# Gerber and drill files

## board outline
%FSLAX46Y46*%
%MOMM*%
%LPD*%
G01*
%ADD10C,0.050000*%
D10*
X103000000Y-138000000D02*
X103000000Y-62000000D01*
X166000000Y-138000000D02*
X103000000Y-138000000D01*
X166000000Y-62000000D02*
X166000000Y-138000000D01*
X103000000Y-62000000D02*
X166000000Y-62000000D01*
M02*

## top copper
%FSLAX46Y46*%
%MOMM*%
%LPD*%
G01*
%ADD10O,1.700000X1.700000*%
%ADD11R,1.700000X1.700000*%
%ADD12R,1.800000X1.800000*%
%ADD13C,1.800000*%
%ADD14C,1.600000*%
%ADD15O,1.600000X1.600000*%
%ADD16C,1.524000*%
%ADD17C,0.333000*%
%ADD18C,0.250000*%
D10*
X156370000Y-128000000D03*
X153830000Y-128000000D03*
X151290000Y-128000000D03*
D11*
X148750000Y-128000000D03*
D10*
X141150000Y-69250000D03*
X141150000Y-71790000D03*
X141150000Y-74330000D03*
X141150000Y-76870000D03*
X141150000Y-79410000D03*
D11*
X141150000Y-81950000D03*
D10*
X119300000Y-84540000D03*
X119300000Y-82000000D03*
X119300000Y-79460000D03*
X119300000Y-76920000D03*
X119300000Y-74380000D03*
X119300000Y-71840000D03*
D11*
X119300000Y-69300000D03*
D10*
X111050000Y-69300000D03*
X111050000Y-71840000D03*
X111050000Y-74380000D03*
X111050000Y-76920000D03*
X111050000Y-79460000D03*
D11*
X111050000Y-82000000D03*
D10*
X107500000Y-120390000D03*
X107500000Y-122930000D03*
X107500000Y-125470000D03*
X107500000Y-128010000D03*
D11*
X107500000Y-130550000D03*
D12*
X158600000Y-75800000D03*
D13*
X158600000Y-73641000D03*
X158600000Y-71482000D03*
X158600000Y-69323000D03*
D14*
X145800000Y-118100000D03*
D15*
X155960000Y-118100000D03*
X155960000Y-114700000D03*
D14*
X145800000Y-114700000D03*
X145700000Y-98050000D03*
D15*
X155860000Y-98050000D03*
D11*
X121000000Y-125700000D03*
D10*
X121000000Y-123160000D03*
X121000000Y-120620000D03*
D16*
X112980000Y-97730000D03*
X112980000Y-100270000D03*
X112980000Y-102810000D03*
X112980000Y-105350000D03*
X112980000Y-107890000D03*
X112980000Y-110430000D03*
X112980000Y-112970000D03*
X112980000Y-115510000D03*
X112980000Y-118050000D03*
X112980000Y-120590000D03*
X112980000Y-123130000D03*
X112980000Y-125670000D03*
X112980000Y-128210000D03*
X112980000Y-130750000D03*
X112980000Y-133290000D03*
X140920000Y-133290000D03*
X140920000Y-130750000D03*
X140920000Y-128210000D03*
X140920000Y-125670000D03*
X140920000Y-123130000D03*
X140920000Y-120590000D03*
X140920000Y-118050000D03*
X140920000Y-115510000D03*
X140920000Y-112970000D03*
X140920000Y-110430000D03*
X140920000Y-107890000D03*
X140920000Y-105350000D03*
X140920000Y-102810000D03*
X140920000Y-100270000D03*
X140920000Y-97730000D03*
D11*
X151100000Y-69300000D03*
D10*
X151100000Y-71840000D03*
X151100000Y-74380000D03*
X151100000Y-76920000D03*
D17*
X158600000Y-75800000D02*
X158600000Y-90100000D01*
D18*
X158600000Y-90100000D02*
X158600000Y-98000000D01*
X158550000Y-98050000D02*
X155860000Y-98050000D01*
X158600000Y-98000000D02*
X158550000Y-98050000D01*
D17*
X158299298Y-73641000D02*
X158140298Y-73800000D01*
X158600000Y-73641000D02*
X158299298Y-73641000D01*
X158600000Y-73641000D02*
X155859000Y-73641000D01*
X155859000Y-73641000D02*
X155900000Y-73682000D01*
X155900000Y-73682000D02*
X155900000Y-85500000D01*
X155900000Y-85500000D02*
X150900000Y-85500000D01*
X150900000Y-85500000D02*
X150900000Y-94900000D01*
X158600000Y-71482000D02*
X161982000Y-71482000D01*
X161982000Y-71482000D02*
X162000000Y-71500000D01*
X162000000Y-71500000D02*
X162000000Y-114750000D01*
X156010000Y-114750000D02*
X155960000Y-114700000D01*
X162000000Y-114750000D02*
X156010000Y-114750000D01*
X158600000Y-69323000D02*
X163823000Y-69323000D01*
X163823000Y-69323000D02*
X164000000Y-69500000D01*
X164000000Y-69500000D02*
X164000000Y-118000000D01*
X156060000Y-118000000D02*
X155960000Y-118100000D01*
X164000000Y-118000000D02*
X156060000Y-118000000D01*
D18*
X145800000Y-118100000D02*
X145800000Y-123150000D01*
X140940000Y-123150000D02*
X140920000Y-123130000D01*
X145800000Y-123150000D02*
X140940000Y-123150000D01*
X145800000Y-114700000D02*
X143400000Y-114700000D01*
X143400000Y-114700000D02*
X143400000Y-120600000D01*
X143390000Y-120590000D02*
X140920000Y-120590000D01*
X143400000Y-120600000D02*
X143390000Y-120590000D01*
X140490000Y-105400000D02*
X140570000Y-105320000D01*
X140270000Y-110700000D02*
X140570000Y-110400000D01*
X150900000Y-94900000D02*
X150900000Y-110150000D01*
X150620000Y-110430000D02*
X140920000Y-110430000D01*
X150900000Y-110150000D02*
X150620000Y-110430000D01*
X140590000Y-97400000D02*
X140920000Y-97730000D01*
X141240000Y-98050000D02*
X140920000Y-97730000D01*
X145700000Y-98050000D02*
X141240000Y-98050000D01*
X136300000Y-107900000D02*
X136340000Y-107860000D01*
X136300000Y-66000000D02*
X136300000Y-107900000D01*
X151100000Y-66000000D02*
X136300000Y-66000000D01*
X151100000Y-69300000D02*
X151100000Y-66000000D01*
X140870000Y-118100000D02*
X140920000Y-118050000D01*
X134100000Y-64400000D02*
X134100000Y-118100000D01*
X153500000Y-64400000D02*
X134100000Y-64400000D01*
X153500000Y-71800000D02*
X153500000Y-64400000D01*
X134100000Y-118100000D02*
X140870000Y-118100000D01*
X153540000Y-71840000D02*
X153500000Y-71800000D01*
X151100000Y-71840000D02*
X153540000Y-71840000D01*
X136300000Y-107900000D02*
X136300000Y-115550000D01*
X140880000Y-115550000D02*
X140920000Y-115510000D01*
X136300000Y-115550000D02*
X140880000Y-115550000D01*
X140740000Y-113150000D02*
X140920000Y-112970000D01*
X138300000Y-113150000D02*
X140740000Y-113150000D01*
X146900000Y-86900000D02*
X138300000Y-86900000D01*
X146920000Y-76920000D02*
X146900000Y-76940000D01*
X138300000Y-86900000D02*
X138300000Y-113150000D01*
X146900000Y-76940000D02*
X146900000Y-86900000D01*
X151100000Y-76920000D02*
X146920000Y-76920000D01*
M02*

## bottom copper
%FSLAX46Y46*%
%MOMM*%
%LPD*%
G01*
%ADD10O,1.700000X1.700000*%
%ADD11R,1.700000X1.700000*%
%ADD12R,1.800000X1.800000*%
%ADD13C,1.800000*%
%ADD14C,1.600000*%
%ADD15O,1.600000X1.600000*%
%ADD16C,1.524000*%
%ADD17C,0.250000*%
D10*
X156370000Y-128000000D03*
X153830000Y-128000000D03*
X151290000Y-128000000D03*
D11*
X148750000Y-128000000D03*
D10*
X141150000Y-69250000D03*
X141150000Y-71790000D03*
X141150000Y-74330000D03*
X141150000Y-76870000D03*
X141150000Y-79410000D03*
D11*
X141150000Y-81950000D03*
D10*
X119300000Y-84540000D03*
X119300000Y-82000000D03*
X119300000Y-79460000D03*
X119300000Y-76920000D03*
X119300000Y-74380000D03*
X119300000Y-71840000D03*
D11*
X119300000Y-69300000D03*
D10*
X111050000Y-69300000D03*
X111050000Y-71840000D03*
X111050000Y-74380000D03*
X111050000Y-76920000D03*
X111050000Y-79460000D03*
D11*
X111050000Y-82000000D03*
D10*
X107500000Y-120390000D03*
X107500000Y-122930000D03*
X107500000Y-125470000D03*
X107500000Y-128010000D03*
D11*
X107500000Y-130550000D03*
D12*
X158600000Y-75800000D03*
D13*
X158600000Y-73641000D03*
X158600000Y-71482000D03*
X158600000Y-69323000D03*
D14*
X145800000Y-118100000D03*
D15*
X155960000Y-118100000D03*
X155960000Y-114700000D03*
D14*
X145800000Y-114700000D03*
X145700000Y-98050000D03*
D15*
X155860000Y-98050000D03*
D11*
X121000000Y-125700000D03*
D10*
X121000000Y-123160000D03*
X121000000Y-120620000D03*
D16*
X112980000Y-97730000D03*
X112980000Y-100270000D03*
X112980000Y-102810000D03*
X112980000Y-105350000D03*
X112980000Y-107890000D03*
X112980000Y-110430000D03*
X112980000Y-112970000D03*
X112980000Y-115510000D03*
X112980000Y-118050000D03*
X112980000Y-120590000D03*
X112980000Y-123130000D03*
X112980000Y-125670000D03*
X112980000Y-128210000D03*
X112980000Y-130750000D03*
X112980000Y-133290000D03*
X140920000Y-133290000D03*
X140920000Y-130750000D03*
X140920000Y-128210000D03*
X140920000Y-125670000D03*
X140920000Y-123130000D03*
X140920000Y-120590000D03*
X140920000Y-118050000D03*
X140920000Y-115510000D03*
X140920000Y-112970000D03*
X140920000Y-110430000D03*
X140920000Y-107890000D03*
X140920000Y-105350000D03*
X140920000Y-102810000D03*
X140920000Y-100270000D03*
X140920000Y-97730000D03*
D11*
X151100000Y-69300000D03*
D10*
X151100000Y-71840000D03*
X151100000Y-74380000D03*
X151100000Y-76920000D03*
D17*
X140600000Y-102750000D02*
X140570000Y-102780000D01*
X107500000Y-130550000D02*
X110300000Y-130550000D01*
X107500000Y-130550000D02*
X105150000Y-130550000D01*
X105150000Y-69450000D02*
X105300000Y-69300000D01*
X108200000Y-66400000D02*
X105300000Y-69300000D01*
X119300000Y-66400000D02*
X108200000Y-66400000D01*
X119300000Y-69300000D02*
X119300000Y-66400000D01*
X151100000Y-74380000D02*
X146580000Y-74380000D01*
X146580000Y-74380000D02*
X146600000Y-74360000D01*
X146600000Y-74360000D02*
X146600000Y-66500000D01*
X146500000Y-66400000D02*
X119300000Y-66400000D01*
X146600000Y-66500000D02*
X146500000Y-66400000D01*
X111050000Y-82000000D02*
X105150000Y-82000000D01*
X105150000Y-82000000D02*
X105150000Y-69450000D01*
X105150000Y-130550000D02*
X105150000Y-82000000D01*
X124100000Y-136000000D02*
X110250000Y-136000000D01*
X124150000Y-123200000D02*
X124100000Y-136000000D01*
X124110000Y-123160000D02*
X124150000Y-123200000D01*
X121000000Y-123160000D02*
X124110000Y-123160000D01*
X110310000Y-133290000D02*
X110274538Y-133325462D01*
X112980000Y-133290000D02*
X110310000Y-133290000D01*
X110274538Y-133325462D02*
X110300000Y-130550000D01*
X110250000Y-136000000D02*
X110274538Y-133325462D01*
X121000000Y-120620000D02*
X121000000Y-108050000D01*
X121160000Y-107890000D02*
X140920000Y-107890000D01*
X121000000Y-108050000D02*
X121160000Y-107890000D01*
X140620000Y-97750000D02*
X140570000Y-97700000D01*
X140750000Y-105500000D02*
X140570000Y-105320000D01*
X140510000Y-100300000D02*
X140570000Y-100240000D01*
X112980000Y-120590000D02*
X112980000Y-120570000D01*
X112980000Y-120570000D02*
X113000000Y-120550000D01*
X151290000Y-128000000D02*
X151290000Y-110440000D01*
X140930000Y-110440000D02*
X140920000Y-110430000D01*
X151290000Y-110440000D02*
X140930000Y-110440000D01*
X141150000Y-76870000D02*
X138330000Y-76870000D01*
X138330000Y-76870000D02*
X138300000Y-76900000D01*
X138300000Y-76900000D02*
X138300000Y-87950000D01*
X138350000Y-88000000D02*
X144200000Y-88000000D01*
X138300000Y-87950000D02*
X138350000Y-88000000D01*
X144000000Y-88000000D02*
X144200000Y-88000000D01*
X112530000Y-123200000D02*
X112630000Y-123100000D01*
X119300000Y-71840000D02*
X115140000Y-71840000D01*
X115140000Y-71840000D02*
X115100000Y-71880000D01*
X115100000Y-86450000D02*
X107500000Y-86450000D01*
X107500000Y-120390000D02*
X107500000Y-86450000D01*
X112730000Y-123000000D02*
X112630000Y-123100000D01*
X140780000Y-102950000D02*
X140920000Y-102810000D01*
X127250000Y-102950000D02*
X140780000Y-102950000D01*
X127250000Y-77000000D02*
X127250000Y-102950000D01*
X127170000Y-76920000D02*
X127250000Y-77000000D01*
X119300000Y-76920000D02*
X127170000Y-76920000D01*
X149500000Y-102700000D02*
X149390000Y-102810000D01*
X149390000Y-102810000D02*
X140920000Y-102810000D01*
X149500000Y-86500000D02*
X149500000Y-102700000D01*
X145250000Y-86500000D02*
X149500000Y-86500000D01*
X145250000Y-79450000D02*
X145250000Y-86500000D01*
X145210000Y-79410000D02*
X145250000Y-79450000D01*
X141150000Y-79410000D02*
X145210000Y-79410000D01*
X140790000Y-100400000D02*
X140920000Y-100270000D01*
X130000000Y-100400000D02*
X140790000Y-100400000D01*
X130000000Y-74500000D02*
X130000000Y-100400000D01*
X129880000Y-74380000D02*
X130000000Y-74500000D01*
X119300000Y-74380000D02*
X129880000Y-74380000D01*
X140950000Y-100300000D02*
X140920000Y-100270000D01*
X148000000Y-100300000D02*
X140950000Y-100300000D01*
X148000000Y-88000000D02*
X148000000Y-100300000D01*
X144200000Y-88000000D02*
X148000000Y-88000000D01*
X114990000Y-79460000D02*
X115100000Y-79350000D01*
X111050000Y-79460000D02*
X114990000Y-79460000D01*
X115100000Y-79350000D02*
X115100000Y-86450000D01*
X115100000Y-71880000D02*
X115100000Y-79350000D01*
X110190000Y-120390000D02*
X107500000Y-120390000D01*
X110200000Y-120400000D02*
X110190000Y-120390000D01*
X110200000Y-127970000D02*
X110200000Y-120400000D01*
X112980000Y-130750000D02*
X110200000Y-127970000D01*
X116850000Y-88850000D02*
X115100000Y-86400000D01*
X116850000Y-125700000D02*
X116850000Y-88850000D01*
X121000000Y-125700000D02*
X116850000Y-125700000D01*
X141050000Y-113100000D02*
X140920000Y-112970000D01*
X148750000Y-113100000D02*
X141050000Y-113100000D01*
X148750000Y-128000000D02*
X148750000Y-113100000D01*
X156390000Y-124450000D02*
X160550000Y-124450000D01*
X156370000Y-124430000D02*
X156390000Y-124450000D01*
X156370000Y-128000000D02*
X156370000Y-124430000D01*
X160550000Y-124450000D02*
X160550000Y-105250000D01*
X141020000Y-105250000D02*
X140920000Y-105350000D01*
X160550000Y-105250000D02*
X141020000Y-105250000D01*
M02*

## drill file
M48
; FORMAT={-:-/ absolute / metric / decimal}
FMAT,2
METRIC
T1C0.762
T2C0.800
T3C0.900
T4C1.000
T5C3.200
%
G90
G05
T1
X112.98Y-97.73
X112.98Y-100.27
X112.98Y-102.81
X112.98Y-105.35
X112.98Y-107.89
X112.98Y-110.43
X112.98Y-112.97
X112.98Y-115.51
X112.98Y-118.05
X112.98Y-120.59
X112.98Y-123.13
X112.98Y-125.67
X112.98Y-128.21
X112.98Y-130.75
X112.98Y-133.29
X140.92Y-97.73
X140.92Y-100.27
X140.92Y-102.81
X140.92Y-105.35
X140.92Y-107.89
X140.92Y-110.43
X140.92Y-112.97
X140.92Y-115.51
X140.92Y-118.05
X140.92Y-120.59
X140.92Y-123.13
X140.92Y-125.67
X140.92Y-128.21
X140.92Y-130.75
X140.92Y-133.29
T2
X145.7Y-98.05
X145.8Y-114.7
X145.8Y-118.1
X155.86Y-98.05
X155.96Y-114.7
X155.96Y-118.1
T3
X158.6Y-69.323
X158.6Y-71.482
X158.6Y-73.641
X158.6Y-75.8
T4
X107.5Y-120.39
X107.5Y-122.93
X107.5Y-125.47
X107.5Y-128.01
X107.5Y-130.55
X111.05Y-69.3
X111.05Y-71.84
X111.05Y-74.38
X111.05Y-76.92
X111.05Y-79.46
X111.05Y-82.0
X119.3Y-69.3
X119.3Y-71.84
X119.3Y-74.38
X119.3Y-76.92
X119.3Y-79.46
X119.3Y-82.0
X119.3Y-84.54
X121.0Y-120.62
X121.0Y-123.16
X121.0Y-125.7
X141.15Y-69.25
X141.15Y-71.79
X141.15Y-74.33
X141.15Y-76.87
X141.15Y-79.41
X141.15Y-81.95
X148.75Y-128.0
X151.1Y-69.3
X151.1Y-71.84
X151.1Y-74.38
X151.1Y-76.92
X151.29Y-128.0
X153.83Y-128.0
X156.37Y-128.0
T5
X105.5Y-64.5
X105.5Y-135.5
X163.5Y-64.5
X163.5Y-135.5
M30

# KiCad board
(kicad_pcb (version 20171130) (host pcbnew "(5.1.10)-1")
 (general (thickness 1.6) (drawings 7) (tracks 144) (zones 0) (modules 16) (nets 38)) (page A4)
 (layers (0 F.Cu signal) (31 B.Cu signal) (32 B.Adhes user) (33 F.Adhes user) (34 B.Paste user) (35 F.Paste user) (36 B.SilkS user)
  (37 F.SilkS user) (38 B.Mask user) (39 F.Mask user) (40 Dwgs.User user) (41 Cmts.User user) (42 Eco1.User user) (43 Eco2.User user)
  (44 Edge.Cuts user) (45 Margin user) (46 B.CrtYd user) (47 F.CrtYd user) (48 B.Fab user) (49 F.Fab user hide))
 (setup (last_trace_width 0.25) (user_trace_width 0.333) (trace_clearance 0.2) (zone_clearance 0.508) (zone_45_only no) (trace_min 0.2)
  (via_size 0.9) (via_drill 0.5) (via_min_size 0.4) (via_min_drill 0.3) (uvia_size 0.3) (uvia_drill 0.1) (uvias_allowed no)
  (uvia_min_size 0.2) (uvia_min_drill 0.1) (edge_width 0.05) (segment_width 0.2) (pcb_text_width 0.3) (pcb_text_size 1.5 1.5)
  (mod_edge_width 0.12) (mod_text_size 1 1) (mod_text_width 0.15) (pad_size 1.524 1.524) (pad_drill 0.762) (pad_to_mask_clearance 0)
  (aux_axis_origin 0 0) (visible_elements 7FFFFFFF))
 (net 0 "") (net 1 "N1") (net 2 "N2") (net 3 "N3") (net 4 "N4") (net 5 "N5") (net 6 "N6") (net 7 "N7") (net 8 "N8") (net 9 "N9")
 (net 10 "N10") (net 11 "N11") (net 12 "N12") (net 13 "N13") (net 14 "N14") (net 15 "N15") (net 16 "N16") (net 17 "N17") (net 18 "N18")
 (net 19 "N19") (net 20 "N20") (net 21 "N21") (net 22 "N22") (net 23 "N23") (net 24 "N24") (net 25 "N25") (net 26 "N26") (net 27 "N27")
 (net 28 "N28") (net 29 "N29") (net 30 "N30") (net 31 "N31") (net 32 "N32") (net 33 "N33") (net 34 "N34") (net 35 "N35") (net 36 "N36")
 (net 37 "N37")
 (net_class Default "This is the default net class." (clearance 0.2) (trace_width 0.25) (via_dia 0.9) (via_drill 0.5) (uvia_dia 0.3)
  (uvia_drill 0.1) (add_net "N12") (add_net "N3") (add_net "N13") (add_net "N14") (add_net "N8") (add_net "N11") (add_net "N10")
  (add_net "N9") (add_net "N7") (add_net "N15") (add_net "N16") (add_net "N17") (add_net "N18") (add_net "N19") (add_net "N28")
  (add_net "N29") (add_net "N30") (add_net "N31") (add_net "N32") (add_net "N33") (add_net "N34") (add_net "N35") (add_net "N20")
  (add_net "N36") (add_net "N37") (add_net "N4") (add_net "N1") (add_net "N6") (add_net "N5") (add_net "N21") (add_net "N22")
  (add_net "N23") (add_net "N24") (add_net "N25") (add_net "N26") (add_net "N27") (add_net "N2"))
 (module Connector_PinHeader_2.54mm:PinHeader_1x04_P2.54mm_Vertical (layer F.Cu) (at 148.75 128 90)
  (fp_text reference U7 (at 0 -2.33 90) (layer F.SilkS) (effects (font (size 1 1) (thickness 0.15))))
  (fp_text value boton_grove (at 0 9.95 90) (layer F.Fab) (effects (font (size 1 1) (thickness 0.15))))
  (pad 4 thru_hole oval (at 0 7.62 90) (size 1.7 1.7) (drill 1) (layers *.Cu *.Mask) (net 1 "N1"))
  (pad 3 thru_hole oval (at 0 5.08 90) (size 1.7 1.7) (drill 1) (layers *.Cu *.Mask) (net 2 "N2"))
  (pad 2 thru_hole oval (at 0 2.54 90) (size 1.7 1.7) (drill 1) (layers *.Cu *.Mask) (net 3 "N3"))
  (pad 1 thru_hole rect (at 0 0 90) (size 1.7 1.7) (drill 1) (layers *.Cu *.Mask) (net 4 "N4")))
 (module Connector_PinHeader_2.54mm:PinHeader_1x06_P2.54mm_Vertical (layer F.Cu) (at 141.15 81.95 180)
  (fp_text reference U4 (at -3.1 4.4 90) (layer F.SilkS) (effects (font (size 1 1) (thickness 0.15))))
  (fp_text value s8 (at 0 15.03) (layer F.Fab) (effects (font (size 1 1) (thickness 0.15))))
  (pad 6 thru_hole oval (at 0 12.7 180) (size 1.7 1.7) (drill 1) (layers *.Cu *.Mask))
  (pad 5 thru_hole oval (at 0 10.16 180) (size 1.7 1.7) (drill 1) (layers *.Cu *.Mask))
  (pad 4 thru_hole oval (at 0 7.62 180) (size 1.7 1.7) (drill 1) (layers *.Cu *.Mask))
  (pad 3 thru_hole oval (at 0 5.08 180) (size 1.7 1.7) (drill 1) (layers *.Cu *.Mask) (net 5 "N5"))
  (pad 2 thru_hole oval (at 0 2.54 180) (size 1.7 1.7) (drill 1) (layers *.Cu *.Mask) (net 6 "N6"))
  (pad 1 thru_hole rect (at 0 0 180) (size 1.7 1.7) (drill 1) (layers *.Cu *.Mask)))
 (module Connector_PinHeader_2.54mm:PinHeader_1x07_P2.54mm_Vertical (layer F.Cu) (at 119.3 69.3)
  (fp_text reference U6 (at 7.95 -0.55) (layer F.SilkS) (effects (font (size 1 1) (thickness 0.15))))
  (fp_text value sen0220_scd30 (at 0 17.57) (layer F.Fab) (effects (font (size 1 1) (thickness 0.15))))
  (pad 7 thru_hole oval (at 0 15.24) (size 1.7 1.7) (drill 1) (layers *.Cu *.Mask))
  (pad 6 thru_hole oval (at 0 12.7) (size 1.7 1.7) (drill 1) (layers *.Cu *.Mask))
  (pad 5 thru_hole oval (at 0 10.16) (size 1.7 1.7) (drill 1) (layers *.Cu *.Mask))
  (pad 4 thru_hole oval (at 0 7.62) (size 1.7 1.7) (drill 1) (layers *.Cu *.Mask) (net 6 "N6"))
  (pad 3 thru_hole oval (at 0 5.08) (size 1.7 1.7) (drill 1) (layers *.Cu *.Mask) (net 5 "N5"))
  (pad 2 thru_hole oval (at 0 2.54) (size 1.7 1.7) (drill 1) (layers *.Cu *.Mask) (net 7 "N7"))
  (pad 1 thru_hole rect (at 0 0) (size 1.7 1.7) (drill 1) (layers *.Cu *.Mask) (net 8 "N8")))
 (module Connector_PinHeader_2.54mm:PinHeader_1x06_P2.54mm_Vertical (layer F.Cu) (at 111.05 82 180)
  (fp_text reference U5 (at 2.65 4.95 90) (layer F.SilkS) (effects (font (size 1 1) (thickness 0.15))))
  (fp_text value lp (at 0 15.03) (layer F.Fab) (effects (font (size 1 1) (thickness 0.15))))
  (pad 6 thru_hole oval (at 0 12.7 180) (size 1.7 1.7) (drill 1) (layers *.Cu *.Mask))
  (pad 5 thru_hole oval (at 0 10.16 180) (size 1.7 1.7) (drill 1) (layers *.Cu *.Mask))
  (pad 4 thru_hole oval (at 0 7.62 180) (size 1.7 1.7) (drill 1) (layers *.Cu *.Mask))
  (pad 3 thru_hole oval (at 0 5.08 180) (size 1.7 1.7) (drill 1) (layers *.Cu *.Mask))
  (pad 2 thru_hole oval (at 0 2.54 180) (size 1.7 1.7) (drill 1) (layers *.Cu *.Mask) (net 7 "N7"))
  (pad 1 thru_hole rect (at 0 0 180) (size 1.7 1.7) (drill 1) (layers *.Cu *.Mask) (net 8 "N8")))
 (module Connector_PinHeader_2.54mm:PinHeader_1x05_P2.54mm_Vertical (layer F.Cu) (at 107.5 130.55 180)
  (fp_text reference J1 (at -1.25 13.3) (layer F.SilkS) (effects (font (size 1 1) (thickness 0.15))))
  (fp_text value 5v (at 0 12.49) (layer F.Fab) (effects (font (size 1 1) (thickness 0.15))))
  (pad 5 thru_hole oval (at 0 10.16 180) (size 1.7 1.7) (drill 1) (layers *.Cu *.Mask) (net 7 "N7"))
  (pad 4 thru_hole oval (at 0 7.62 180) (size 1.7 1.7) (drill 1) (layers *.Cu *.Mask) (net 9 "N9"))
  (pad 3 thru_hole oval (at 0 5.08 180) (size 1.7 1.7) (drill 1) (layers *.Cu *.Mask) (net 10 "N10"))
  (pad 2 thru_hole oval (at 0 2.54 180) (size 1.7 1.7) (drill 1) (layers *.Cu *.Mask) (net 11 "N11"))
  (pad 1 thru_hole rect (at 0 0 180) (size 1.7 1.7) (drill 1) (layers *.Cu *.Mask) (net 8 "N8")))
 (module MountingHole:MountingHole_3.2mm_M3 (layer F.Cu) (at 105.5 64.5)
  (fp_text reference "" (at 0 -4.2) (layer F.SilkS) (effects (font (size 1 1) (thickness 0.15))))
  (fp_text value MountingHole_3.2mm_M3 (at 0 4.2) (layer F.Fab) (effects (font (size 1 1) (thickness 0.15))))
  (pad 1 np_thru_hole circle (at 0 0) (size 3.2 3.2) (drill 3.2) (layers *.Cu *.Mask)))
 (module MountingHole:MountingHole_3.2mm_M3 (layer F.Cu) (at 105.5 135.5)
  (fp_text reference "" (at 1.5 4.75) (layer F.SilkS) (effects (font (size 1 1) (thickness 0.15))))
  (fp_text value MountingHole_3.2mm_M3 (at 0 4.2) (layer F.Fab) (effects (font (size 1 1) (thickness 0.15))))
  (pad 1 np_thru_hole circle (at 0 0) (size 3.2 3.2) (drill 3.2) (layers *.Cu *.Mask)))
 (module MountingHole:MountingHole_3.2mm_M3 (layer F.Cu) (at 163.5 135.5)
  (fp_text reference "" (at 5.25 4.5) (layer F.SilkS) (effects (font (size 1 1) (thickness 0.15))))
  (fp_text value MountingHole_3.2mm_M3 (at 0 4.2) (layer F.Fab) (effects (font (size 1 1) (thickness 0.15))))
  (pad 1 np_thru_hole circle (at 0 0) (size 3.2 3.2) (drill 3.2) (layers *.Cu *.Mask)))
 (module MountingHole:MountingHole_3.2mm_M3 (layer F.Cu) (at 163.5 64.5)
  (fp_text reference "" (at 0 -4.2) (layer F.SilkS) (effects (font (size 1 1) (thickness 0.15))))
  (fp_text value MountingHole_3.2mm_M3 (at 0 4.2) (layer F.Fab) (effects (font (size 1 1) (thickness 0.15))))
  (pad 1 np_thru_hole circle (at 0 0) (size 3.2 3.2) (drill 3.2) (layers *.Cu *.Mask)))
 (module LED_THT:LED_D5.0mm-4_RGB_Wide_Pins (layer F.Cu) (at 158.6 75.8 90)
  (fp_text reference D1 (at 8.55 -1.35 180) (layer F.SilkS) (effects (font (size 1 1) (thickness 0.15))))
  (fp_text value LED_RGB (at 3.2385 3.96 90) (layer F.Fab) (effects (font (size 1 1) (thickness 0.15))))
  (pad 1 thru_hole rect (at 0 0 90) (size 1.8 1.8) (drill 0.9) (layers *.Cu *.Mask) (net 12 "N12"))
  (pad 2 thru_hole circle (at 2.159 0 90) (size 1.8 1.8) (drill 0.9) (layers *.Cu *.Mask) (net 3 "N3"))
  (pad 3 thru_hole circle (at 4.318 0 90) (size 1.8 1.8) (drill 0.9) (layers *.Cu *.Mask) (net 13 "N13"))
  (pad 4 thru_hole circle (at 6.477 0 90) (size 1.8 1.8) (drill 0.9) (layers *.Cu *.Mask) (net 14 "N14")))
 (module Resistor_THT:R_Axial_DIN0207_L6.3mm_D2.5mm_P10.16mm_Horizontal (layer F.Cu) (at 145.8 118.1)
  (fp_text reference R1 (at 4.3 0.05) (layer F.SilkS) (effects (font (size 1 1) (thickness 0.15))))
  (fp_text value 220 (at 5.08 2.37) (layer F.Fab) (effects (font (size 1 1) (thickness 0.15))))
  (pad 1 thru_hole circle (at 0 0) (size 1.6 1.6) (drill 0.8) (layers *.Cu *.Mask) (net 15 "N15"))
  (pad 2 thru_hole oval (at 10.16 0) (size 1.6 1.6) (drill 0.8) (layers *.Cu *.Mask) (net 14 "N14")))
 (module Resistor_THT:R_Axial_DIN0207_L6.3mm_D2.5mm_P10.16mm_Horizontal (layer F.Cu) (at 145.8 114.7)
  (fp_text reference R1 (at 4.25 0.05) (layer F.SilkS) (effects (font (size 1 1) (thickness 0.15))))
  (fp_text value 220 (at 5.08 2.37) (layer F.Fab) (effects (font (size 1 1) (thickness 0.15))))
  (pad 2 thru_hole oval (at 10.16 0) (size 1.6 1.6) (drill 0.8) (layers *.Cu *.Mask) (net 13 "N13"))
  (pad 1 thru_hole circle (at 0 0) (size 1.6 1.6) (drill 0.8) (layers *.Cu *.Mask) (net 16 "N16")))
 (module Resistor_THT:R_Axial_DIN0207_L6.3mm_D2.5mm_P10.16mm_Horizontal (layer F.Cu) (at 145.7 98.05)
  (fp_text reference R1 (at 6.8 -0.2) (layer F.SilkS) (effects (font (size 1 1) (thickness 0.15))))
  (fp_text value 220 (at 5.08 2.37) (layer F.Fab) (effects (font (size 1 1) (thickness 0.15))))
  (pad 1 thru_hole circle (at 0 0) (size 1.6 1.6) (drill 0.8) (layers *.Cu *.Mask) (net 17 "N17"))
  (pad 2 thru_hole oval (at 10.16 0) (size 1.6 1.6) (drill 0.8) (layers *.Cu *.Mask) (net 12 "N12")))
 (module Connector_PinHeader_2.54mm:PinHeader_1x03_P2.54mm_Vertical (layer F.Cu) (at 121 125.7 180)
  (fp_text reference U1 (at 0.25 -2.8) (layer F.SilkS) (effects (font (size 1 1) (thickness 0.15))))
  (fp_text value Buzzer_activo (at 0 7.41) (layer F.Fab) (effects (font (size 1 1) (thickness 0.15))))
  (pad 1 thru_hole rect (at 0 0 180) (size 1.7 1.7) (drill 1) (layers *.Cu *.Mask) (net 7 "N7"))
  (pad 2 thru_hole oval (at 0 2.54 180) (size 1.7 1.7) (drill 1) (layers *.Cu *.Mask) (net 8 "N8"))
  (pad 3 thru_hole oval (at 0 5.08 180) (size 1.7 1.7) (drill 1) (layers *.Cu *.Mask) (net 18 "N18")))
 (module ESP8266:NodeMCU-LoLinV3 (layer F.Cu) (at 126.95 118.05)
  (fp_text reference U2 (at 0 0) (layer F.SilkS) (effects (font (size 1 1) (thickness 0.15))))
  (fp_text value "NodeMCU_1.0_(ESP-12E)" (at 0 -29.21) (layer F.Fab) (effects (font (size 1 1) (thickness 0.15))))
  (pad 1 thru_hole circle (at -13.97 -20.32) (size 1.524 1.524) (drill 0.762) (layers *.Cu *.Mask F.SilkS) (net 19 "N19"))
  (pad 2 thru_hole circle (at -13.97 -17.78) (size 1.524 1.524) (drill 0.762) (layers *.Cu *.Mask F.SilkS) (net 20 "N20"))
  (pad 3 thru_hole circle (at -13.97 -15.24) (size 1.524 1.524) (drill 0.762) (layers *.Cu *.Mask F.SilkS) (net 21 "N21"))
  (pad 4 thru_hole circle (at -13.97 -12.7) (size 1.524 1.524) (drill 0.762) (layers *.Cu *.Mask F.SilkS) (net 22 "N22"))
  (pad 5 thru_hole circle (at -13.97 -10.16) (size 1.524 1.524) (drill 0.762) (layers *.Cu *.Mask F.SilkS) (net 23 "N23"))
  (pad 6 thru_hole circle (at -13.97 -7.62) (size 1.524 1.524) (drill 0.762) (layers *.Cu *.Mask F.SilkS) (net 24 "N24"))
  (pad 7 thru_hole circle (at -13.97 -5.08) (size 1.524 1.524) (drill 0.762) (layers *.Cu *.Mask F.SilkS) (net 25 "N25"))
  (pad 8 thru_hole circle (at -13.97 -2.54) (size 1.524 1.524) (drill 0.762) (layers *.Cu *.Mask F.SilkS) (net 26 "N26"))
  (pad 9 thru_hole circle (at -13.97 0) (size 1.524 1.524) (drill 0.762) (layers *.Cu *.Mask F.SilkS) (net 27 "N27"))
  (pad 10 thru_hole circle (at -13.97 2.54) (size 1.524 1.524) (drill 0.762) (layers *.Cu *.Mask F.SilkS) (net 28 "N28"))
  (pad 11 thru_hole circle (at -13.97 5.08) (size 1.524 1.524) (drill 0.762) (layers *.Cu *.Mask F.SilkS) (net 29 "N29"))
  (pad 12 thru_hole circle (at -13.97 7.62) (size 1.524 1.524) (drill 0.762) (layers *.Cu *.Mask F.SilkS) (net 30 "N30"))
  (pad 13 thru_hole circle (at -13.97 10.16) (size 1.524 1.524) (drill 0.762) (layers *.Cu *.Mask F.SilkS) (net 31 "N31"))
  (pad 14 thru_hole circle (at -13.97 12.7) (size 1.524 1.524) (drill 0.762) (layers *.Cu *.Mask F.SilkS) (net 7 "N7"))
  (pad 15 thru_hole circle (at -13.97 15.24) (size 1.524 1.524) (drill 0.762) (layers *.Cu *.Mask F.SilkS) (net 8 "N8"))
  (pad 16 thru_hole circle (at 13.97 15.24) (size 1.524 1.524) (drill 0.762) (layers *.Cu *.Mask F.SilkS) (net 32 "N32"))
  (pad 17 thru_hole circle (at 13.97 12.7) (size 1.524 1.524) (drill 0.762) (layers *.Cu *.Mask F.SilkS) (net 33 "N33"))
  (pad 18 thru_hole circle (at 13.97 10.16) (size 1.524 1.524) (drill 0.762) (layers *.Cu *.Mask F.SilkS) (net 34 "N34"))
  (pad 19 thru_hole circle (at 13.97 7.62) (size 1.524 1.524) (drill 0.762) (layers *.Cu *.Mask F.SilkS) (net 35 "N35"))
  (pad 20 thru_hole circle (at 13.97 5.08) (size 1.524 1.524) (drill 0.762) (layers *.Cu *.Mask F.SilkS) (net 15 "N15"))
  (pad 21 thru_hole circle (at 13.97 2.54) (size 1.524 1.524) (drill 0.762) (layers *.Cu *.Mask F.SilkS) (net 16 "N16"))
  (pad 22 thru_hole circle (at 13.97 0) (size 1.524 1.524) (drill 0.762) (layers *.Cu *.Mask F.SilkS) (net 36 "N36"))
  (pad 23 thru_hole circle (at 13.97 -2.54) (size 1.524 1.524) (drill 0.762) (layers *.Cu *.Mask F.SilkS) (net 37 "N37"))
  (pad 24 thru_hole circle (at 13.97 -5.08) (size 1.524 1.524) (drill 0.762) (layers *.Cu *.Mask F.SilkS) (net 4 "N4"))
  (pad 25 thru_hole circle (at 13.97 -7.62) (size 1.524 1.524) (drill 0.762) (layers *.Cu *.Mask F.SilkS) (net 3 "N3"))
  (pad 26 thru_hole circle (at 13.97 -10.16) (size 1.524 1.524) (drill 0.762) (layers *.Cu *.Mask F.SilkS) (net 18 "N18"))
  (pad 27 thru_hole circle (at 13.97 -12.7) (size 1.524 1.524) (drill 0.762) (layers *.Cu *.Mask F.SilkS) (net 1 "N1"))
  (pad 28 thru_hole circle (at 13.97 -15.24) (size 1.524 1.524) (drill 0.762) (layers *.Cu *.Mask F.SilkS) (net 6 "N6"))
  (pad 29 thru_hole circle (at 13.97 -17.78) (size 1.524 1.524) (drill 0.762) (layers *.Cu *.Mask F.SilkS) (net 5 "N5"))
  (pad 30 thru_hole circle (at 13.97 -20.32) (size 1.524 1.524) (drill 0.762) (layers *.Cu *.Mask F.SilkS) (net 17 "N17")))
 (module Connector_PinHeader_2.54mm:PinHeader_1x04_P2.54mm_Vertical (layer F.Cu) (at 151.1 69.3)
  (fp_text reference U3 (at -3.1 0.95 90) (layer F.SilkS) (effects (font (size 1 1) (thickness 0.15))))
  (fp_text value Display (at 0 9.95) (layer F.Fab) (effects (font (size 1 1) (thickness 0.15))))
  (pad 1 thru_hole rect (at 0 0) (size 1.7 1.7) (drill 1) (layers *.Cu *.Mask) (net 37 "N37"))
  (pad 2 thru_hole oval (at 0 2.54) (size 1.7 1.7) (drill 1) (layers *.Cu *.Mask) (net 36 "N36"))
  (pad 3 thru_hole oval (at 0 5.08) (size 1.7 1.7) (drill 1) (layers *.Cu *.Mask) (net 8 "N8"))
  (pad 4 thru_hole oval (at 0 7.62) (size 1.7 1.7) (drill 1) (layers *.Cu *.Mask) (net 4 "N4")))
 (gr_line (start 103 138) (end 103 62) (layer Edge.Cuts) (width 0.05))
 (gr_line (start 166 138) (end 103 138) (layer Edge.Cuts) (width 0.05))
 (gr_line (start 166 62) (end 166 138) (layer Edge.Cuts) (width 0.05))
 (gr_line (start 103 62) (end 166 62) (layer Edge.Cuts) (width 0.05))
 (segment (start 158.6 75.8) (end 158.6 90.1) (width 0.333) (layer F.Cu) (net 12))
 (segment (start 158.6 90.1) (end 158.6 98) (width 0.25) (layer F.Cu) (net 12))
 (segment (start 158.55 98.05) (end 155.86 98.05) (width 0.25) (layer F.Cu) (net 12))
 (segment (start 158.6 98) (end 158.55 98.05) (width 0.25) (layer F.Cu) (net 12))
 (segment (start 158.299298 73.641) (end 158.140298 73.8) (width 0.333) (layer F.Cu) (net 3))
 (segment (start 158.6 73.641) (end 158.299298 73.641) (width 0.333) (layer F.Cu) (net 3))
 (segment (start 158.6 73.641) (end 155.859 73.641) (width 0.333) (layer F.Cu) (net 3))
 (segment (start 155.859 73.641) (end 155.9 73.682) (width 0.333) (layer F.Cu) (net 3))
 (segment (start 155.9 73.682) (end 155.9 85.5) (width 0.333) (layer F.Cu) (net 3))
 (segment (start 155.9 85.5) (end 150.9 85.5) (width 0.333) (layer F.Cu) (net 3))
 (segment (start 150.9 85.5) (end 150.9 94.9) (width 0.333) (layer F.Cu) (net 3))
 (segment (start 140.6 102.75) (end 140.57 102.78) (width 0.25) (layer B.Cu) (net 6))
 (segment (start 158.6 71.482) (end 161.982 71.482) (width 0.333) (layer F.Cu) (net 13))
 (segment (start 161.982 71.482) (end 162 71.5) (width 0.333) (layer F.Cu) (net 13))
 (segment (start 162 71.5) (end 162 114.75) (width 0.333) (layer F.Cu) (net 13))
 (segment (start 156.01 114.75) (end 155.96 114.7) (width 0.333) (layer F.Cu) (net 13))
 (segment (start 162 114.75) (end 156.01 114.75) (width 0.333) (layer F.Cu) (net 13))
 (segment (start 158.6 69.323) (end 163.823 69.323) (width 0.333) (layer F.Cu) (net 14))
 (segment (start 163.823 69.323) (end 164 69.5) (width 0.333) (layer F.Cu) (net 14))
 (segment (start 164 69.5) (end 164 118) (width 0.333) (layer F.Cu) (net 14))
 (segment (start 156.06 118) (end 155.96 118.1) (width 0.333) (layer F.Cu) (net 14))
 (segment (start 164 118) (end 156.06 118) (width 0.333) (layer F.Cu) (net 14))
 (segment (start 107.5 130.55) (end 110.3 130.55) (width 0.25) (layer B.Cu) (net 8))
 (segment (start 107.5 130.55) (end 105.15 130.55) (width 0.25) (layer B.Cu) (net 8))
 (segment (start 105.15 69.45) (end 105.3 69.3) (width 0.25) (layer B.Cu) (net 8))
 (segment (start 108.2 66.4) (end 105.3 69.3) (width 0.25) (layer B.Cu) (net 8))
 (segment (start 119.3 66.4) (end 108.2 66.4) (width 0.25) (layer B.Cu) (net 8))
 (segment (start 119.3 69.3) (end 119.3 66.4) (width 0.25) (layer B.Cu) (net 8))
 (segment (start 151.1 74.38) (end 146.58 74.38) (width 0.25) (layer B.Cu) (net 8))
 (segment (start 146.58 74.38) (end 146.6 74.36) (width 0.25) (layer B.Cu) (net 8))
 (segment (start 146.6 74.36) (end 146.6 66.5) (width 0.25) (layer B.Cu) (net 8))
 (segment (start 146.5 66.4) (end 119.3 66.4) (width 0.25) (layer B.Cu) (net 8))
 (segment (start 146.6 66.5) (end 146.5 66.4) (width 0.25) (layer B.Cu) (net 8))
 (segment (start 111.05 82) (end 105.15 82) (width 0.25) (layer B.Cu) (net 8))
 (segment (start 105.15 82) (end 105.15 69.45) (width 0.25) (layer B.Cu) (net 8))
 (segment (start 105.15 130.55) (end 105.15 82) (width 0.25) (layer B.Cu) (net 8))
 (segment (start 124.1 136) (end 110.25 136) (width 0.25) (layer B.Cu) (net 8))
 (segment (start 124.15 123.2) (end 124.1 136) (width 0.25) (layer B.Cu) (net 8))
 (segment (start 124.11 123.16) (end 124.15 123.2) (width 0.25) (layer B.Cu) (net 8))
 (segment (start 121 123.16) (end 124.11 123.16) (width 0.25) (layer B.Cu) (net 8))
 (segment (start 110.31 133.29) (end 110.274538 133.325462) (width 0.25) (layer B.Cu) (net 8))
 (segment (start 112.98 133.29) (end 110.31 133.29) (width 0.25) (layer B.Cu) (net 8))
 (segment (start 110.274538 133.325462) (end 110.3 130.55) (width 0.25) (layer B.Cu) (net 8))
 (segment (start 110.25 136) (end 110.274538 133.325462) (width 0.25) (layer B.Cu) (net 8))
 (segment (start 145.8 118.1) (end 145.8 123.15) (width 0.25) (layer F.Cu) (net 15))
 (segment (start 140.94 123.15) (end 140.92 123.13) (width 0.25) (layer F.Cu) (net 15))
 (segment (start 145.8 123.15) (end 140.94 123.15) (width 0.25) (layer F.Cu) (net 15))
 (segment (start 145.8 114.7) (end 143.4 114.7) (width 0.25) (layer F.Cu) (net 16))
 (segment (start 143.4 114.7) (end 143.4 120.6) (width 0.25) (layer F.Cu) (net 16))
 (segment (start 143.39 120.59) (end 140.92 120.59) (width 0.25) (layer F.Cu) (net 16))
 (segment (start 143.4 120.6) (end 143.39 120.59) (width 0.25) (layer F.Cu) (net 16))
 (segment (start 121 120.62) (end 121 108.05) (width 0.25) (layer B.Cu) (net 18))
 (segment (start 121.16 107.89) (end 140.92 107.89) (width 0.25) (layer B.Cu) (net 18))
 (segment (start 121 108.05) (end 121.16 107.89) (width 0.25) (layer B.Cu) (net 18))
 (segment (start 140.62 97.75) (end 140.57 97.7) (width 0.25) (layer B.Cu) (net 17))
 (segment (start 140.49 105.4) (end 140.57 105.32) (width 0.25) (layer F.Cu) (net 1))
 (segment (start 140.75 105.5) (end 140.57 105.32) (width 0.25) (layer B.Cu) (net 1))
 (segment (start 140.51 100.3) (end 140.57 100.24) (width 0.25) (layer B.Cu) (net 5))
 (segment (start 112.98 120.59) (end 112.98 120.57) (width 0.25) (layer B.Cu) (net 28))
 (segment (start 112.98 120.57) (end 113 120.55) (width 0.25) (layer B.Cu) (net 28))
 (segment (start 140.27 110.7) (end 140.57 110.4) (width 0.25) (layer F.Cu) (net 3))
 (segment (start 150.9 94.9) (end 150.9 110.15) (width 0.25) (layer F.Cu) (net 3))
 (segment (start 150.62 110.43) (end 140.92 110.43) (width 0.25) (layer F.Cu) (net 3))
 (segment (start 150.9 110.15) (end 150.62 110.43) (width 0.25) (layer F.Cu) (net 3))
 (segment (start 151.29 128) (end 151.29 110.44) (width 0.25) (layer B.Cu) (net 3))
 (segment (start 140.93 110.44) (end 140.92 110.43) (width 0.25) (layer B.Cu) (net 3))
 (segment (start 151.29 110.44) (end 140.93 110.44) (width 0.25) (layer B.Cu) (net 3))
 (segment (start 140.59 97.4) (end 140.92 97.73) (width 0.25) (layer F.Cu) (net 17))
 (segment (start 141.24 98.05) (end 140.92 97.73) (width 0.25) (layer F.Cu) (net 17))
 (segment (start 145.7 98.05) (end 141.24 98.05) (width 0.25) (layer F.Cu) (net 17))
 (segment (start 136.3 107.9) (end 136.34 107.86) (width 0.25) (layer F.Cu) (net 37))
 (segment (start 136.3 66) (end 136.3 107.9) (width 0.25) (layer F.Cu) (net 37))
 (segment (start 151.1 66) (end 136.3 66) (width 0.25) (layer F.Cu) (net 37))
 (segment (start 151.1 69.3) (end 151.1 66) (width 0.25) (layer F.Cu) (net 37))
 (segment (start 141.15 76.87) (end 138.33 76.87) (width 0.25) (layer B.Cu) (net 5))
 (segment (start 138.33 76.87) (end 138.3 76.9) (width 0.25) (layer B.Cu) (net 5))
 (segment (start 138.3 76.9) (end 138.3 87.95) (width 0.25) (layer B.Cu) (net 5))
 (segment (start 138.35 88) (end 144.2 88) (width 0.25) (layer B.Cu) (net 5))
 (segment (start 138.3 87.95) (end 138.35 88) (width 0.25) (layer B.Cu) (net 5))
 (segment (start 144 88) (end 144.2 88) (width 0.25) (layer B.Cu) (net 5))
 (segment (start 112.53 123.2) (end 112.63 123.1) (width 0.25) (layer B.Cu) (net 29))
 (segment (start 119.3 71.84) (end 115.14 71.84) (width 0.25) (layer B.Cu) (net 7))
 (segment (start 115.14 71.84) (end 115.1 71.88) (width 0.25) (layer B.Cu) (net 7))
 (segment (start 115.1 86.45) (end 107.5 86.45) (width 0.25) (layer B.Cu) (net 7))
 (segment (start 107.5 120.39) (end 107.5 86.45) (width 0.25) (layer B.Cu) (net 7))
 (segment (start 112.73 123) (end 112.63 123.1) (width 0.25) (layer B.Cu) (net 29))
 (segment (start 140.87 118.1) (end 140.92 118.05) (width 0.25) (layer F.Cu) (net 36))
 (segment (start 134.1 64.4) (end 134.1 118.1) (width 0.25) (layer F.Cu) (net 36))
 (segment (start 153.5 64.4) (end 134.1 64.4) (width 0.25) (layer F.Cu) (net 36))
 (segment (start 153.5 71.8) (end 153.5 64.4) (width 0.25) (layer F.Cu) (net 36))
 (segment (start 134.1 118.1) (end 140.87 118.1) (width 0.25) (layer F.Cu) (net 36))
 (segment (start 153.54 71.84) (end 153.5 71.8) (width 0.25) (layer F.Cu) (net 36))
 (segment (start 151.1 71.84) (end 153.54 71.84) (width 0.25) (layer F.Cu) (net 36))
 (segment (start 136.3 107.9) (end 136.3 115.55) (width 0.25) (layer F.Cu) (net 37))
 (segment (start 140.88 115.55) (end 140.92 115.51) (width 0.25) (layer F.Cu) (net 37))
 (segment (start 136.3 115.55) (end 140.88 115.55) (width 0.25) (layer F.Cu) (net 37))
 (segment (start 140.78 102.95) (end 140.92 102.81) (width 0.25) (layer B.Cu) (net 6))
 (segment (start 127.25 102.95) (end 140.78 102.95) (width 0.25) (layer B.Cu) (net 6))
 (segment (start 127.25 77) (end 127.25 102.95) (width 0.25) (layer B.Cu) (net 6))
 (segment (start 127.17 76.92) (end 127.25 77) (width 0.25) (layer B.Cu) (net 6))
 (segment (start 119.3 76.92) (end 127.17 76.92) (width 0.25) (layer B.Cu) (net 6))
 (segment (start 149.5 102.7) (end 149.39 102.81) (width 0.25) (layer B.Cu) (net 6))
 (segment (start 149.39 102.81) (end 140.92 102.81) (width 0.25) (layer B.Cu) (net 6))
 (segment (start 149.5 86.5) (end 149.5 102.7) (width 0.25) (layer B.Cu) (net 6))
 (segment (start 145.25 86.5) (end 149.5 86.5) (width 0.25) (layer B.Cu) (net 6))
 (segment (start 145.25 79.45) (end 145.25 86.5) (width 0.25) (layer B.Cu) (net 6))
 (segment (start 145.21 79.41) (end 145.25 79.45) (width 0.25) (layer B.Cu) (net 6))
 (segment (start 141.15 79.41) (end 145.21 79.41) (width 0.25) (layer B.Cu) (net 6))
 (segment (start 140.79 100.4) (end 140.92 100.27) (width 0.25) (layer B.Cu) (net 5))
 (segment (start 130 100.4) (end 140.79 100.4) (width 0.25) (layer B.Cu) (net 5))
 (segment (start 130 74.5) (end 130 100.4) (width 0.25) (layer B.Cu) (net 5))
 (segment (start 129.88 74.38) (end 130 74.5) (width 0.25) (layer B.Cu) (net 5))
 (segment (start 119.3 74.38) (end 129.88 74.38) (width 0.25) (layer B.Cu) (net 5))
 (segment (start 140.95 100.3) (end 140.92 100.27) (width 0.25) (layer B.Cu) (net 5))
 (segment (start 148 100.3) (end 140.95 100.3) (width 0.25) (layer B.Cu) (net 5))
 (segment (start 148 88) (end 148 100.3) (width 0.25) (layer B.Cu) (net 5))
 (segment (start 144.2 88) (end 148 88) (width 0.25) (layer B.Cu) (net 5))
 (segment (start 114.99 79.46) (end 115.1 79.35) (width 0.25) (layer B.Cu) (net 7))
 (segment (start 111.05 79.46) (end 114.99 79.46) (width 0.25) (layer B.Cu) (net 7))
 (segment (start 115.1 79.35) (end 115.1 86.45) (width 0.25) (layer B.Cu) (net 7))
 (segment (start 115.1 71.88) (end 115.1 79.35) (width 0.25) (layer B.Cu) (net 7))
 (segment (start 110.19 120.39) (end 107.5 120.39) (width 0.25) (layer B.Cu) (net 7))
 (segment (start 110.2 120.4) (end 110.19 120.39) (width 0.25) (layer B.Cu) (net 7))
 (segment (start 110.2 127.97) (end 110.2 120.4) (width 0.25) (layer B.Cu) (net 7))
 (segment (start 112.98 130.75) (end 110.2 127.97) (width 0.25) (layer B.Cu) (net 7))
 (segment (start 116.85 88.85) (end 115.1 86.4) (width 0.25) (layer B.Cu) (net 7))
 (segment (start 116.85 125.7) (end 116.85 88.85) (width 0.25) (layer B.Cu) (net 7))
 (segment (start 121 125.7) (end 116.85 125.7) (width 0.25) (layer B.Cu) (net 7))
 (segment (start 140.74 113.15) (end 140.92 112.97) (width 0.25) (layer F.Cu) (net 4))
 (segment (start 138.3 113.15) (end 140.74 113.15) (width 0.25) (layer F.Cu) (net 4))
 (segment (start 146.9 86.9) (end 138.3 86.9) (width 0.25) (layer F.Cu) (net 4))
 (segment (start 146.92 76.92) (end 146.9 76.94) (width 0.25) (layer F.Cu) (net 4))
 (segment (start 138.3 86.9) (end 138.3 113.15) (width 0.25) (layer F.Cu) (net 4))
 (segment (start 146.9 76.94) (end 146.9 86.9) (width 0.25) (layer F.Cu) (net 4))
 (segment (start 151.1 76.92) (end 146.92 76.92) (width 0.25) (layer F.Cu) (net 4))
 (segment (start 141.05 113.1) (end 140.92 112.97) (width 0.25) (layer B.Cu) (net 4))
 (segment (start 148.75 113.1) (end 141.05 113.1) (width 0.25) (layer B.Cu) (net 4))
 (segment (start 148.75 128) (end 148.75 113.1) (width 0.25) (layer B.Cu) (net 4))
 (segment (start 156.39 124.45) (end 160.55 124.45) (width 0.25) (layer B.Cu) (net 1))
 (segment (start 156.37 124.43) (end 156.39 124.45) (width 0.25) (layer B.Cu) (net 1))
 (segment (start 156.37 128) (end 156.37 124.43) (width 0.25) (layer B.Cu) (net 1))
 (segment (start 160.55 124.45) (end 160.55 105.25) (width 0.25) (layer B.Cu) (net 1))
 (segment (start 141.02 105.25) (end 140.92 105.35) (width 0.25) (layer B.Cu) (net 1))
 (segment (start 160.55 105.25) (end 141.02 105.25) (width 0.25) (layer B.Cu) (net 1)))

